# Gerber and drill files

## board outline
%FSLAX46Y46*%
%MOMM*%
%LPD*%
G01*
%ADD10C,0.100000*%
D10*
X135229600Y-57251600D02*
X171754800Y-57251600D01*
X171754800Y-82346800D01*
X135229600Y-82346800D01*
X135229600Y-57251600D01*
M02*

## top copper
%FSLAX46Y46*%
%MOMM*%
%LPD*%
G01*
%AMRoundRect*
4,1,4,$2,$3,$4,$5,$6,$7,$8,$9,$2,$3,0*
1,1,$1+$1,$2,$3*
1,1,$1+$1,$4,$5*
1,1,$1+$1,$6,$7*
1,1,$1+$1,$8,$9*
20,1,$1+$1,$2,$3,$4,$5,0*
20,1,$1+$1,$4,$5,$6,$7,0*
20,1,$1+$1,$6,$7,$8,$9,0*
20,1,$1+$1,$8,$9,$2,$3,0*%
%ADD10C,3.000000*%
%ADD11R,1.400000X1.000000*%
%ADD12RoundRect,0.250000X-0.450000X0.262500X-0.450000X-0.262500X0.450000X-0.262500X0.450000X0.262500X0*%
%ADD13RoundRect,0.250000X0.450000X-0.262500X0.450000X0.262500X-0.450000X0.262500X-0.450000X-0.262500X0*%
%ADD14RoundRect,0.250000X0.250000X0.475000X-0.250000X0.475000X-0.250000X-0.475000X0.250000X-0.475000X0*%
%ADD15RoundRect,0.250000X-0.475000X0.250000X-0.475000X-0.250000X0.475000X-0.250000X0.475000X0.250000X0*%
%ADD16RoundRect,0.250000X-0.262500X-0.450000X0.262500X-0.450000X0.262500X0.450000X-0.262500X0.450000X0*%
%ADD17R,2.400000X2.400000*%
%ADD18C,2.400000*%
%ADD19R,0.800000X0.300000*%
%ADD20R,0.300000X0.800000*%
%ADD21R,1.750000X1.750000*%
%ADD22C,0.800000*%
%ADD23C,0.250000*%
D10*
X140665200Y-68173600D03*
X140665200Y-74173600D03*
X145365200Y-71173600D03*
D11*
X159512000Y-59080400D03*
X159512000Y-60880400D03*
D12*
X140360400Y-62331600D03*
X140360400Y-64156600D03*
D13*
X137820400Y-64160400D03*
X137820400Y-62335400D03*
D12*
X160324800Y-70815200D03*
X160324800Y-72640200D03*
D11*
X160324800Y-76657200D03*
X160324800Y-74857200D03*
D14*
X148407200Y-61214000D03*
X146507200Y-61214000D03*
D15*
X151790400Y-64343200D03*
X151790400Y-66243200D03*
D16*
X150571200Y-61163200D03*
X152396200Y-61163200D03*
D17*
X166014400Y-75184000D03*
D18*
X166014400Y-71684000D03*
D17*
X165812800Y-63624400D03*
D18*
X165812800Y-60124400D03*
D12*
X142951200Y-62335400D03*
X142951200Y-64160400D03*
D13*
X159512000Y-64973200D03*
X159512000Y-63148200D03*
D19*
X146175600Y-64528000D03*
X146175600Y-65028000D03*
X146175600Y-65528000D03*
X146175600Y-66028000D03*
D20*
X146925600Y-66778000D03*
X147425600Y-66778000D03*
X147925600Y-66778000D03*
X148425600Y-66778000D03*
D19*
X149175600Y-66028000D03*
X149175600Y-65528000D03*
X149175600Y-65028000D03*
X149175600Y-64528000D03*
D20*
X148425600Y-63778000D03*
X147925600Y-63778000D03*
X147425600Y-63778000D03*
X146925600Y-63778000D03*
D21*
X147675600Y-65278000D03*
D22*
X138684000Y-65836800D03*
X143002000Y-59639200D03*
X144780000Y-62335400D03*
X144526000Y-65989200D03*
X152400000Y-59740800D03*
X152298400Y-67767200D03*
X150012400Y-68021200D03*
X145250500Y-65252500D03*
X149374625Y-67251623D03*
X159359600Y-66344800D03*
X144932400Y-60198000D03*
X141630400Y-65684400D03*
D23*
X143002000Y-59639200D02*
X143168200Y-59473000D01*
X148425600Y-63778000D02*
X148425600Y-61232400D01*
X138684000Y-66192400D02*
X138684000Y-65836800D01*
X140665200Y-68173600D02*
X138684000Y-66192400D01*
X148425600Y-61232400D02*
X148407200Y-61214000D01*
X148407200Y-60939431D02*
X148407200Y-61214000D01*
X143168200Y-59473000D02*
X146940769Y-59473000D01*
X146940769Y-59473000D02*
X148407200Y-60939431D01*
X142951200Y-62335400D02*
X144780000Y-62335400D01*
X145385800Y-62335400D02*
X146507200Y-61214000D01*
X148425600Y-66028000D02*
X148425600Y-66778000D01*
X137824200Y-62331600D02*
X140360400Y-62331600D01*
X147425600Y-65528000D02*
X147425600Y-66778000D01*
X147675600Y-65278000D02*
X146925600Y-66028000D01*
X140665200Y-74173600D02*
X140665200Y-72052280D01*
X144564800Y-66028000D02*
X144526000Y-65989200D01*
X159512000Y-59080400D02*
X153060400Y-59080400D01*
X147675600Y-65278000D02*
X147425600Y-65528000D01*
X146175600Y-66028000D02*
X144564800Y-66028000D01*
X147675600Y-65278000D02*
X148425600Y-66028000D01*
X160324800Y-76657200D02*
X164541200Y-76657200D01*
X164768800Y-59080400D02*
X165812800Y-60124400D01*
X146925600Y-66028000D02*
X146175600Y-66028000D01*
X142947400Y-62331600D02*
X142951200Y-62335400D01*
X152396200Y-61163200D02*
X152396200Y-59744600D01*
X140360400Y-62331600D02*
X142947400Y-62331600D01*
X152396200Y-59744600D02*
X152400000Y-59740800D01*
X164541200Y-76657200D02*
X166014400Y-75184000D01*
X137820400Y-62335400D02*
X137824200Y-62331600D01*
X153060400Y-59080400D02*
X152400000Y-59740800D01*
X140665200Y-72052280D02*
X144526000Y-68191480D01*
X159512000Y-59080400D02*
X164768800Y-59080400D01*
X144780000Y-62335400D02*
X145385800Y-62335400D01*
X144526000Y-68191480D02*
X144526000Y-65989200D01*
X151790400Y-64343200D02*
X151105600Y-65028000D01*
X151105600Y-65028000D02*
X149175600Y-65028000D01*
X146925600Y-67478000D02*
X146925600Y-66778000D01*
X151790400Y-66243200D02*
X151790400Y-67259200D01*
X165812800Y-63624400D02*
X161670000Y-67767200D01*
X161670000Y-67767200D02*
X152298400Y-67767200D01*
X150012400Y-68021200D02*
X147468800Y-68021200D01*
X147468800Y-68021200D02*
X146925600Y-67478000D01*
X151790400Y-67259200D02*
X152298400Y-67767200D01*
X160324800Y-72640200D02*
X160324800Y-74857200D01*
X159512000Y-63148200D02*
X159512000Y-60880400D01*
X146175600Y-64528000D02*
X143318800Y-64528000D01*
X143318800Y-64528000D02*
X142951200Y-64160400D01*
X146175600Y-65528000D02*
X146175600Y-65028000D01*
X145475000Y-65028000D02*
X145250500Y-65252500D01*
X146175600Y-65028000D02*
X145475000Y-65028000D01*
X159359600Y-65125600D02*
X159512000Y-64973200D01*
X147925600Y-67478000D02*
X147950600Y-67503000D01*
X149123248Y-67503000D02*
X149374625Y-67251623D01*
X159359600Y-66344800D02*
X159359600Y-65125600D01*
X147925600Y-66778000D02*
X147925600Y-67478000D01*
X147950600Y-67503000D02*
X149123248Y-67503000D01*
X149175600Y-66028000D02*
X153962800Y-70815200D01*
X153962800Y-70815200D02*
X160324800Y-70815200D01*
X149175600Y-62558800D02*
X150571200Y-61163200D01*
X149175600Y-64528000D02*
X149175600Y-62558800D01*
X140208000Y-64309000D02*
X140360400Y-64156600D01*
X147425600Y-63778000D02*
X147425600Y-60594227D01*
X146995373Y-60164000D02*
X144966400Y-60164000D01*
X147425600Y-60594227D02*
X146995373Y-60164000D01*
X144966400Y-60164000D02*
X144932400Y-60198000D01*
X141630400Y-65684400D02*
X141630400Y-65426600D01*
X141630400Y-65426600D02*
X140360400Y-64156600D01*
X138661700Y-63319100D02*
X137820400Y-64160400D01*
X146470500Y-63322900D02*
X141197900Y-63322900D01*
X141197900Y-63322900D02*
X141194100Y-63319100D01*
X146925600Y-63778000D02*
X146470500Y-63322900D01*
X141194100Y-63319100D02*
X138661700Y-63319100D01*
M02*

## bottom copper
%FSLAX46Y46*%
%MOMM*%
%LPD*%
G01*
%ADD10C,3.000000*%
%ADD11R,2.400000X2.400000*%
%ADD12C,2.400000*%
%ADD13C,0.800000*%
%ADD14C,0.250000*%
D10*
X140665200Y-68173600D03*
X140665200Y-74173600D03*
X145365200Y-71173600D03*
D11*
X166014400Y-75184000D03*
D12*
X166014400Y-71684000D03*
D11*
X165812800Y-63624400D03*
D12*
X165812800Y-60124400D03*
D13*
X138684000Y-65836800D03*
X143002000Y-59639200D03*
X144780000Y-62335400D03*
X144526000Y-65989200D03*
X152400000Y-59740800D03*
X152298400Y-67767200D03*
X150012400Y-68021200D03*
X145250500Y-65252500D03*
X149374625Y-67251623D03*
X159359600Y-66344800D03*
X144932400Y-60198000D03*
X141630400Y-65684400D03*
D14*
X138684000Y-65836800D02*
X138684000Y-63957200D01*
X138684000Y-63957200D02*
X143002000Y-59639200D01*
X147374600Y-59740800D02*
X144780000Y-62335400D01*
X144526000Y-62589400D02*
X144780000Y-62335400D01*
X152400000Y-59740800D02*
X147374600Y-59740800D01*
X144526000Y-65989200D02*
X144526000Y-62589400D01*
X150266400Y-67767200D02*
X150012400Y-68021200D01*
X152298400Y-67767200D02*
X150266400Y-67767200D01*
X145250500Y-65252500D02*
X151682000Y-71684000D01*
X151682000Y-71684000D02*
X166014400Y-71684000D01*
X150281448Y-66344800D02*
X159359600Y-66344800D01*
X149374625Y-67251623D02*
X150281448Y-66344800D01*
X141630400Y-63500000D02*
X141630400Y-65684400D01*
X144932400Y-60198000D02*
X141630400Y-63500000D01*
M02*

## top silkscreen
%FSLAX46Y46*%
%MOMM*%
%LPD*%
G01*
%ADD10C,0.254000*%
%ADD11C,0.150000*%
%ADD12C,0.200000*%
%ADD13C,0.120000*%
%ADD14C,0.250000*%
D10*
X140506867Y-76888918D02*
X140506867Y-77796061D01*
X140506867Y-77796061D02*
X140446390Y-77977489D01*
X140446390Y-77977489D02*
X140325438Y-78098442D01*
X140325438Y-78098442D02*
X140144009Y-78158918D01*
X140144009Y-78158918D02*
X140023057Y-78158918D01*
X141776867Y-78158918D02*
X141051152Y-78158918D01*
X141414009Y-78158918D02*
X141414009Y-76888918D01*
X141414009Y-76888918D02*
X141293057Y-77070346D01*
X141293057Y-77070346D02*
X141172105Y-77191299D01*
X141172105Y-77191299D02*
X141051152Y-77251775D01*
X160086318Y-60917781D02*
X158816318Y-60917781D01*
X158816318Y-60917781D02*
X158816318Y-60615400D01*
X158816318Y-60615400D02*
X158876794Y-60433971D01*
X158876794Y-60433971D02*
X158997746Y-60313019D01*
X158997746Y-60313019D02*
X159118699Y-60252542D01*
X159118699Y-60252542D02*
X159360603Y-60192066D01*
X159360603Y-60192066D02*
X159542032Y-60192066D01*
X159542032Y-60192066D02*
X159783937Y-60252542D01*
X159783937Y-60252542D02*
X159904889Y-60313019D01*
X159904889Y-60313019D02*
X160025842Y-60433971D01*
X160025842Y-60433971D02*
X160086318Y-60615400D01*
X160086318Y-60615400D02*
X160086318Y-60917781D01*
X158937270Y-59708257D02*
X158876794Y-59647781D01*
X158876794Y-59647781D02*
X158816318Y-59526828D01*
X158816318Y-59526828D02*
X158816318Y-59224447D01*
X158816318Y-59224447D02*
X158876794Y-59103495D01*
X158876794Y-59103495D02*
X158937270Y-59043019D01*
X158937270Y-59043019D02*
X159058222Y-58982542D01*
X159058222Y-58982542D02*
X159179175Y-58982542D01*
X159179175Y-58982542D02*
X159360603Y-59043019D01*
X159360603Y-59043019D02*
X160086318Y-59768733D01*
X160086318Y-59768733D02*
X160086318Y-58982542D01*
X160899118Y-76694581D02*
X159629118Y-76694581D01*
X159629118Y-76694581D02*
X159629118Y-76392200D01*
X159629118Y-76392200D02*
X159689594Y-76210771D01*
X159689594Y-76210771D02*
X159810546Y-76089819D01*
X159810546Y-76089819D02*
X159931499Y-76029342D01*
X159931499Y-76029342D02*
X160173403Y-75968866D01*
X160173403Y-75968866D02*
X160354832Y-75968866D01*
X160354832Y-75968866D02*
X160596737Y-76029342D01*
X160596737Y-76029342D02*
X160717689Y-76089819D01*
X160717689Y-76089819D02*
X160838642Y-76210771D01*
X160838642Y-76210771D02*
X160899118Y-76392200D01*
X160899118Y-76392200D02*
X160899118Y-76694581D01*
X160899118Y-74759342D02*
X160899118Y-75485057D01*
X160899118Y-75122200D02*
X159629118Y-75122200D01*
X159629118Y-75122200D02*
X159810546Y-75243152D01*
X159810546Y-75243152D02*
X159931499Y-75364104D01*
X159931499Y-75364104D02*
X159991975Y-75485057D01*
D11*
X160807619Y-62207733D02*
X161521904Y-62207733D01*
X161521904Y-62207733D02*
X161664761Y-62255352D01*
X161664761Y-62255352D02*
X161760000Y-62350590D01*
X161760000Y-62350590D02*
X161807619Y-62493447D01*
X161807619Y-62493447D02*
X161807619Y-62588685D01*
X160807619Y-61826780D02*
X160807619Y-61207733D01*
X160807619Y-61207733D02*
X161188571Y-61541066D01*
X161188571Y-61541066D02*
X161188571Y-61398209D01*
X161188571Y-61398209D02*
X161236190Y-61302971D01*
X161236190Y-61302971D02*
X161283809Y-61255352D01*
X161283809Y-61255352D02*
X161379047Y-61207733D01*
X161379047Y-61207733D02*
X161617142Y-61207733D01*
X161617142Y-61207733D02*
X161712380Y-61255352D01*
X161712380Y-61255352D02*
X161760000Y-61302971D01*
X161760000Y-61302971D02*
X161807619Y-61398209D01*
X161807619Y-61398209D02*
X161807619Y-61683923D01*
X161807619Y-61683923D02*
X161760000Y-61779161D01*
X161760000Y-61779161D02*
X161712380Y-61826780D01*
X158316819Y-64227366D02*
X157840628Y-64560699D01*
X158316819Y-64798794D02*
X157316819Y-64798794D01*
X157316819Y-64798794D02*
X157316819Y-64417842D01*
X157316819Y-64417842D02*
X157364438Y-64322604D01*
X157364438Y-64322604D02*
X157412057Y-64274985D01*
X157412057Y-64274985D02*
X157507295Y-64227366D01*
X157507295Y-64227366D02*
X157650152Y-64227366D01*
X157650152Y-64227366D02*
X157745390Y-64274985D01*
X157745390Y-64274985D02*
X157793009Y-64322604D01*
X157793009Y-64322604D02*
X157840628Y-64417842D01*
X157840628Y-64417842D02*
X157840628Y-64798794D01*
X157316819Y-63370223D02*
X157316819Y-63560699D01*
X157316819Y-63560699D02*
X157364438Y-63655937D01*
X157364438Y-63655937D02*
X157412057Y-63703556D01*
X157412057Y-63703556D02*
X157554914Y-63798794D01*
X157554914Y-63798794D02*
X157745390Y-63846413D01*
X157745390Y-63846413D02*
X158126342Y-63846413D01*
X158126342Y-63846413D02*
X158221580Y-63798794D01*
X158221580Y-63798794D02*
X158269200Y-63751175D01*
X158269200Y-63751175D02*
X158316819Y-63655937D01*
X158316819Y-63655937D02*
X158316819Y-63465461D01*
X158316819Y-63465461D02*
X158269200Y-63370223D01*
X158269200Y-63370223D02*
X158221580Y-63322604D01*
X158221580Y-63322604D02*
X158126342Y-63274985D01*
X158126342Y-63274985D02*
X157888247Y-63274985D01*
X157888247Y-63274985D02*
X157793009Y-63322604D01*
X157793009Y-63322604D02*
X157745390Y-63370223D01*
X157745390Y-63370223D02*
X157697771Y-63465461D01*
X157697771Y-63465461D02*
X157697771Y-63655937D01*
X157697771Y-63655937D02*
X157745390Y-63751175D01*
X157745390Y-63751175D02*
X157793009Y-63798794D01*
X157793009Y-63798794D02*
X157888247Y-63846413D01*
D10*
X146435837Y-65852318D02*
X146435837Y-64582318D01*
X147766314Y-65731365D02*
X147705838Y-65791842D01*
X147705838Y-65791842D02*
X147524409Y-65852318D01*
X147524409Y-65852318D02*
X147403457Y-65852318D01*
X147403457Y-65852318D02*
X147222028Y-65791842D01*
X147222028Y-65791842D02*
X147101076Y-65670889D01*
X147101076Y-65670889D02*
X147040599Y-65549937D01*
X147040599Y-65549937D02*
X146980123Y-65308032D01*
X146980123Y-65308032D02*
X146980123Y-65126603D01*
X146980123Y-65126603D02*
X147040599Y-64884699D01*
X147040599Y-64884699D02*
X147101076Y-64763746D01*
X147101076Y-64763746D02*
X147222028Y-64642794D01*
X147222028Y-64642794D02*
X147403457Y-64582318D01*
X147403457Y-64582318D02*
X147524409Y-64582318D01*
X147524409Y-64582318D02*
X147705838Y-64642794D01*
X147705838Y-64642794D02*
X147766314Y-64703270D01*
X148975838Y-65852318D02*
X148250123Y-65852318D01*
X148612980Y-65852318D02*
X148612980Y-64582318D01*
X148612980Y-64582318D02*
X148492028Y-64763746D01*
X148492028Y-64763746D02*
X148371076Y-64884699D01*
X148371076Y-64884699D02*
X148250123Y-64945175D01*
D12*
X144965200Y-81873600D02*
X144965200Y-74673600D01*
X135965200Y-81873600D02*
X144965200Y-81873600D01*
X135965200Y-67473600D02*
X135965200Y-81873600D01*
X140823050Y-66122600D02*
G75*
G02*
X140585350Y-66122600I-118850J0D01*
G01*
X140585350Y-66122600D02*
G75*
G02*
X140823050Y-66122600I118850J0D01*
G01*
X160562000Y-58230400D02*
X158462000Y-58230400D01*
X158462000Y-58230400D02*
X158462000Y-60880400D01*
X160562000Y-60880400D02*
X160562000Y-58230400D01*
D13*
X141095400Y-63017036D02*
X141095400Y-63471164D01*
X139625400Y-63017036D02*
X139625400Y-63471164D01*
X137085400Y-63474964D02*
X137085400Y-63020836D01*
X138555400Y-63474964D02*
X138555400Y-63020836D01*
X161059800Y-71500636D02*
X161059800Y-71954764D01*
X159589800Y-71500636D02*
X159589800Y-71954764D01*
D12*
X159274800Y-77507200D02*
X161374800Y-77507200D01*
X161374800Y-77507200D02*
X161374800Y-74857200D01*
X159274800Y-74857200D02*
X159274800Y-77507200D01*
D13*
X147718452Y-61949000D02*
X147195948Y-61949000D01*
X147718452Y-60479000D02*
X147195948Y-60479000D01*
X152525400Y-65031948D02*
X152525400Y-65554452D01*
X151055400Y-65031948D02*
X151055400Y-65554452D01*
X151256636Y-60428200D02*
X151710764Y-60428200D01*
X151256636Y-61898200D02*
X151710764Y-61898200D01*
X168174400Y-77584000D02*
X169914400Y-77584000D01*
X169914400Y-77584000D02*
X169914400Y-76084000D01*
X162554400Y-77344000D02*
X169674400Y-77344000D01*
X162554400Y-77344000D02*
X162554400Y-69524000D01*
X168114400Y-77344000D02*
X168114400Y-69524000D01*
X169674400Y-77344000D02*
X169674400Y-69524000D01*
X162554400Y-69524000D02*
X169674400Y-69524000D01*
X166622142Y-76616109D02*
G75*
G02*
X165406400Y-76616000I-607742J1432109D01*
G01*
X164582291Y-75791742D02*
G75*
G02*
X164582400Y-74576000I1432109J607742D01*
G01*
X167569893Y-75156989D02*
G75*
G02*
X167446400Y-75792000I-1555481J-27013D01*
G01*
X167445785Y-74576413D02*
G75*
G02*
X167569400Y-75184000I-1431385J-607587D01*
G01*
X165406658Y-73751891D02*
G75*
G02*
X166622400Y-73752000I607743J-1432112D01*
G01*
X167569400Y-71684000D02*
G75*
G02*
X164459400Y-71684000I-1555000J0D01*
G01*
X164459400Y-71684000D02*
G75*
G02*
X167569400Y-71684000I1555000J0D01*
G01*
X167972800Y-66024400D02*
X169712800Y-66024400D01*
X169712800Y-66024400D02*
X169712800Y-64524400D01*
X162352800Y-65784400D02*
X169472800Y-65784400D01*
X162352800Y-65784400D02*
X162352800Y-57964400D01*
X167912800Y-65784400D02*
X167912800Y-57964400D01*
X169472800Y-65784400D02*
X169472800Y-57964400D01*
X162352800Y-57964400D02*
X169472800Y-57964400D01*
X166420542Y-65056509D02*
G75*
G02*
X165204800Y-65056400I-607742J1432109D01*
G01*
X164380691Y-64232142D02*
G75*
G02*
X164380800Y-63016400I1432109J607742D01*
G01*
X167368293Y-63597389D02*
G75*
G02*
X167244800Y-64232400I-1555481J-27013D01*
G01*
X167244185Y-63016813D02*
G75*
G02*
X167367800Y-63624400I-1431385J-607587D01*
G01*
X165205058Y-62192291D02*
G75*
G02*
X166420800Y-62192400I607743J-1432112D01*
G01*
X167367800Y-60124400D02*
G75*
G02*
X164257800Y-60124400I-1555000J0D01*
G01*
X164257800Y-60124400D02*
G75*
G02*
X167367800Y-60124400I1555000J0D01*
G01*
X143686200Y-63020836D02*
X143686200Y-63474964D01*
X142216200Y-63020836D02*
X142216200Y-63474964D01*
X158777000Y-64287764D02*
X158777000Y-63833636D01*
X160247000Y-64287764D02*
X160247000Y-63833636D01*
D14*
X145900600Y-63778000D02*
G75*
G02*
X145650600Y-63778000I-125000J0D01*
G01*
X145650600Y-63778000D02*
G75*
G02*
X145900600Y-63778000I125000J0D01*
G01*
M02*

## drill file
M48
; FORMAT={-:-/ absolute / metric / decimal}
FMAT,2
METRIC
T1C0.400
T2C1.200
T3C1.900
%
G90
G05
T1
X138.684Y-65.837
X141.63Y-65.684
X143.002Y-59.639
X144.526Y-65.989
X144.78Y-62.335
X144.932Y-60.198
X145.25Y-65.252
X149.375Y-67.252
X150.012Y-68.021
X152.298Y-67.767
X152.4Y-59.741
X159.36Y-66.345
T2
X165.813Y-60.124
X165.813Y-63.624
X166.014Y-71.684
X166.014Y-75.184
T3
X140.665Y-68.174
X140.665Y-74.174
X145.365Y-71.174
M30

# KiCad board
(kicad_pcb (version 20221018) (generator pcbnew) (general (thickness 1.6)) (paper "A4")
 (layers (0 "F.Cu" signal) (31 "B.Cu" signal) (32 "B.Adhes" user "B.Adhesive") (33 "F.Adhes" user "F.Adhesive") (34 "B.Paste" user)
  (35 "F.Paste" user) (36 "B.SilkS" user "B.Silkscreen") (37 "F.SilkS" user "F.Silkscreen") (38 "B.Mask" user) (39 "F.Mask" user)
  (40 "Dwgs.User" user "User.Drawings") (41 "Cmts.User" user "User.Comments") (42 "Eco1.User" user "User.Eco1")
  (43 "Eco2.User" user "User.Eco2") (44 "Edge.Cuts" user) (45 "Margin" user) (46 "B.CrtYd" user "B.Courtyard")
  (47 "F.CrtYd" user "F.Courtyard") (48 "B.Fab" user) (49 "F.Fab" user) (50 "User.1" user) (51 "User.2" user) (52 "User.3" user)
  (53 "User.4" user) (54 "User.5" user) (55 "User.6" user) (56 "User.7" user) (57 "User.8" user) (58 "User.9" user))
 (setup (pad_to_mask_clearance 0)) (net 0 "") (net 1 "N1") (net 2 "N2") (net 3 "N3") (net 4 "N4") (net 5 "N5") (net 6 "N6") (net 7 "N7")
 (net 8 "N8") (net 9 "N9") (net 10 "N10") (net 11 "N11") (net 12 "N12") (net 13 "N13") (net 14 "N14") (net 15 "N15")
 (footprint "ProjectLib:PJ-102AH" (layer "F.Cu") (at 144.9652 71.1736 180)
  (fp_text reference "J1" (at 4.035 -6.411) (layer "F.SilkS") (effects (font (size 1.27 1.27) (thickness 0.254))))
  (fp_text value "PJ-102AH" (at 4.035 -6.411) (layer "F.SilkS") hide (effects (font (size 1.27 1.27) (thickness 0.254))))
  (fp_line (start 0 -10.7) (end 0 -3.5) (stroke (width 0.2) (type solid)) (layer "F.SilkS"))
  (fp_line (start 9 -10.7) (end 0 -10.7) (stroke (width 0.2) (type solid)) (layer "F.SilkS"))
  (fp_line (start 9 3.7) (end 9 -10.7) (stroke (width 0.2) (type solid)) (layer "F.SilkS"))
  (fp_circle (center 4.261 5.051) (end 4.261 5.16985) (stroke (width 0.2) (type solid)) (fill none) (layer "F.SilkS"))
  (pad "1" thru_hole circle (at 4.3 3 180) (size 3 3) (drill 1.9) (layers "*.Cu" "*.Mask") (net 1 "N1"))
  (pad "2" thru_hole circle (at 4.3 -3 180) (size 3 3) (drill 1.9) (layers "*.Cu" "*.Mask") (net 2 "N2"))
  (pad "3" thru_hole circle (at -0.4 0 180) (size 3 3) (drill 1.9) (layers "*.Cu" "*.Mask") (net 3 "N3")))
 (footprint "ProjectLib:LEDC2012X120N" (layer "F.Cu") (at 159.512 59.9804 -90)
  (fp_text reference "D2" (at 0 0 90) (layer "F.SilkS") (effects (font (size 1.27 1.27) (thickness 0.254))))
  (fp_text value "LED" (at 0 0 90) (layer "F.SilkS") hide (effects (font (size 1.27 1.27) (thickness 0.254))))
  (fp_line (start -1.75 -1.05) (end -1.75 1.05) (stroke (width 0.2) (type solid)) (layer "F.SilkS"))
  (fp_line (start -1.75 1.05) (end 0.9 1.05) (stroke (width 0.2) (type solid)) (layer "F.SilkS"))
  (fp_line (start 0.9 -1.05) (end -1.75 -1.05) (stroke (width 0.2) (type solid)) (layer "F.SilkS"))
  (pad "1" smd rect (at -0.9 0 270) (size 1 1.4) (layers "F.Cu" "F.Paste" "F.Mask") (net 2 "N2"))
  (pad "2" smd rect (at 0.9 0 270) (size 1 1.4) (layers "F.Cu" "F.Paste" "F.Mask") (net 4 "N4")))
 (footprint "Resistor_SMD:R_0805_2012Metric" (layer "F.Cu") (at 140.3604 63.2441 -90)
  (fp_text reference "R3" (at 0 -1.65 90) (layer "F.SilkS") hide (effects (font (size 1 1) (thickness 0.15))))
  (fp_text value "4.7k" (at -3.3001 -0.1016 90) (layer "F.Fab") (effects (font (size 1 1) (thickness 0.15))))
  (fp_line (start -0.227064 -0.735) (end 0.227064 -0.735) (stroke (width 0.12) (type solid)) (layer "F.SilkS"))
  (fp_line (start -0.227064 0.735) (end 0.227064 0.735) (stroke (width 0.12) (type solid)) (layer "F.SilkS"))
  (pad "1" smd roundrect (at -0.9125 0 270) (size 1.025 1.4) (layers "F.Cu" "F.Paste" "F.Mask") (roundrect_rratio 0.243902) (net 2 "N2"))
  (pad "2" smd roundrect (at 0.9125 0 270) (size 1.025 1.4) (layers "F.Cu" "F.Paste" "F.Mask") (roundrect_rratio 0.243902) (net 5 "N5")))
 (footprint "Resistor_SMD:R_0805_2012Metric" (layer "F.Cu") (at 137.8204 63.2479 90)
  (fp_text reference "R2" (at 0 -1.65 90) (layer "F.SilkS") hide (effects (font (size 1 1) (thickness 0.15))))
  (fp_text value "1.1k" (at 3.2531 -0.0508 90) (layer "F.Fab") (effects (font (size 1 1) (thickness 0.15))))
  (fp_line (start -0.227064 -0.735) (end 0.227064 -0.735) (stroke (width 0.12) (type solid)) (layer "F.SilkS"))
  (fp_line (start -0.227064 0.735) (end 0.227064 0.735) (stroke (width 0.12) (type solid)) (layer "F.SilkS"))
  (pad "1" smd roundrect (at -0.9125 0 90) (size 1.025 1.4) (layers "F.Cu" "F.Paste" "F.Mask") (roundrect_rratio 0.243902) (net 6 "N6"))
  (pad "2" smd roundrect (at 0.9125 0 90) (size 1.025 1.4) (layers "F.Cu" "F.Paste" "F.Mask") (roundrect_rratio 0.243902) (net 2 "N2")))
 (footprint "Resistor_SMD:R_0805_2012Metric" (layer "F.Cu") (at 160.3248 71.7277 -90)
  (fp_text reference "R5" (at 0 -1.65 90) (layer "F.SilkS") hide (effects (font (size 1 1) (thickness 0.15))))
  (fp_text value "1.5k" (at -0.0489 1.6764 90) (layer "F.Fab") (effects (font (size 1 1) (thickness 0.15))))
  (fp_line (start -0.227064 -0.735) (end 0.227064 -0.735) (stroke (width 0.12) (type solid)) (layer "F.SilkS"))
  (fp_line (start -0.227064 0.735) (end 0.227064 0.735) (stroke (width 0.12) (type solid)) (layer "F.SilkS"))
  (pad "1" smd roundrect (at -0.9125 0 270) (size 1.025 1.4) (layers "F.Cu" "F.Paste" "F.Mask") (roundrect_rratio 0.243902) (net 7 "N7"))
  (pad "2" smd roundrect (at 0.9125 0 270) (size 1.025 1.4) (layers "F.Cu" "F.Paste" "F.Mask") (roundrect_rratio 0.243902) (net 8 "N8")))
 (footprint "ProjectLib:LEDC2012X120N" (layer "F.Cu") (at 160.3248 75.7572 90)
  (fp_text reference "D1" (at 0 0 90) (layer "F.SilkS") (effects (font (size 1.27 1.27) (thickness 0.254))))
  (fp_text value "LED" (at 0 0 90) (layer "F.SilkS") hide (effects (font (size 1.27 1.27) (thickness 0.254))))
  (fp_line (start -1.75 -1.05) (end -1.75 1.05) (stroke (width 0.2) (type solid)) (layer "F.SilkS"))
  (fp_line (start -1.75 1.05) (end 0.9 1.05) (stroke (width 0.2) (type solid)) (layer "F.SilkS"))
  (fp_line (start 0.9 -1.05) (end -1.75 -1.05) (stroke (width 0.2) (type solid)) (layer "F.SilkS"))
  (pad "1" smd rect (at -0.9 0 90) (size 1 1.4) (layers "F.Cu" "F.Paste" "F.Mask") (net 2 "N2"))
  (pad "2" smd rect (at 0.9 0 90) (size 1 1.4) (layers "F.Cu" "F.Paste" "F.Mask") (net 8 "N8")))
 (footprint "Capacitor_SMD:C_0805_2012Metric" (layer "F.Cu") (at 147.4572 61.214 180)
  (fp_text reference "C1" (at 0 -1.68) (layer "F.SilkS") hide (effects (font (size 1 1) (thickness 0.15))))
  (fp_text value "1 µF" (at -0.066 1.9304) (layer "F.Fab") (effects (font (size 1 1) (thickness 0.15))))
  (fp_line (start -0.261252 -0.735) (end 0.261252 -0.735) (stroke (width 0.12) (type solid)) (layer "F.SilkS"))
  (fp_line (start -0.261252 0.735) (end 0.261252 0.735) (stroke (width 0.12) (type solid)) (layer "F.SilkS"))
  (pad "1" smd roundrect (at -0.95 0 180) (size 1 1.45) (layers "F.Cu" "F.Paste" "F.Mask") (roundrect_rratio 0.25) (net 1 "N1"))
  (pad "2" smd roundrect (at 0.95 0 180) (size 1 1.45) (layers "F.Cu" "F.Paste" "F.Mask") (roundrect_rratio 0.25) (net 2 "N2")))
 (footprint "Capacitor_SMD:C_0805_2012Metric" (layer "F.Cu") (at 151.7904 65.2932 -90)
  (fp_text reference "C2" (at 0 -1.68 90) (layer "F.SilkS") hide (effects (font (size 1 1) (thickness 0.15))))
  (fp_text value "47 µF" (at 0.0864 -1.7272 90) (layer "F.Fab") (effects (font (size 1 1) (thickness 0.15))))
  (fp_line (start -0.261252 -0.735) (end 0.261252 -0.735) (stroke (width 0.12) (type solid)) (layer "F.SilkS"))
  (fp_line (start -0.261252 0.735) (end 0.261252 0.735) (stroke (width 0.12) (type solid)) (layer "F.SilkS"))
  (pad "1" smd roundrect (at -0.95 0 270) (size 1 1.45) (layers "F.Cu" "F.Paste" "F.Mask") (roundrect_rratio 0.25) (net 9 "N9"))
  (pad "2" smd roundrect (at 0.95 0 270) (size 1 1.45) (layers "F.Cu" "F.Paste" "F.Mask") (roundrect_rratio 0.25) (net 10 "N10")))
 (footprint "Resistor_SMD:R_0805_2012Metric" (layer "F.Cu") (at 151.4837 61.1632)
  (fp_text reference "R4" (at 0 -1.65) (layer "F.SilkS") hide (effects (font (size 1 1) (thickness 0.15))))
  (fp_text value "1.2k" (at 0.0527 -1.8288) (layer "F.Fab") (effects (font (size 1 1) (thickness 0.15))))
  (fp_line (start -0.227064 -0.735) (end 0.227064 -0.735) (stroke (width 0.12) (type solid)) (layer "F.SilkS"))
  (fp_line (start -0.227064 0.735) (end 0.227064 0.735) (stroke (width 0.12) (type solid)) (layer "F.SilkS"))
  (pad "1" smd roundrect (at -0.9125 0) (size 1.025 1.4) (layers "F.Cu" "F.Paste" "F.Mask") (roundrect_rratio 0.243902) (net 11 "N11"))
  (pad "2" smd roundrect (at 0.9125 0) (size 1.025 1.4) (layers "F.Cu" "F.Paste" "F.Mask") (roundrect_rratio 0.243902) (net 2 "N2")))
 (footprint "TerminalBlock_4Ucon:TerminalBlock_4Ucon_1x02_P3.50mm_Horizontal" (layer "F.Cu") (at 166.0144 75.184 90)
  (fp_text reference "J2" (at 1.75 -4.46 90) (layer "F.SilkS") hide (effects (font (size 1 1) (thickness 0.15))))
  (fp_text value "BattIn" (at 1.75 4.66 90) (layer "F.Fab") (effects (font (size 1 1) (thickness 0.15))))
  (fp_line (start -2.4 2.16) (end -2.4 3.9) (stroke (width 0.12) (type solid)) (layer "F.SilkS"))
  (fp_line (start -2.4 3.9) (end -0.9 3.9) (stroke (width 0.12) (type solid)) (layer "F.SilkS"))
  (fp_line (start -2.16 -3.46) (end -2.16 3.66) (stroke (width 0.12) (type solid)) (layer "F.SilkS"))
  (fp_line (start -2.16 -3.46) (end 5.66 -3.46) (stroke (width 0.12) (type solid)) (layer "F.SilkS"))
  (fp_line (start -2.16 2.1) (end 5.66 2.1) (stroke (width 0.12) (type solid)) (layer "F.SilkS"))
  (fp_line (start -2.16 3.66) (end 5.66 3.66) (stroke (width 0.12) (type solid)) (layer "F.SilkS"))
  (fp_line (start 5.66 -3.46) (end 5.66 3.66) (stroke (width 0.12) (type solid)) (layer "F.SilkS"))
  (fp_arc (start -1.432109 0.607742) (mid -1.555727 -0.00014) (end -1.432 -0.608) (stroke (width 0.12) (type solid)) (layer "F.SilkS"))
  (fp_arc (start -0.607742 -1.432109) (mid 0.00014 -1.555727) (end 0.608 -1.432) (stroke (width 0.12) (type solid)) (layer "F.SilkS"))
  (fp_arc (start 0.027011 1.555493) (mid -0.296984 1.527118) (end -0.608 1.432) (stroke (width 0.12) (type solid)) (layer "F.SilkS"))
  (fp_arc (start 0.607587 1.431385) (mid 0.310017 1.523783) (end 0 1.555) (stroke (width 0.12) (type solid)) (layer "F.SilkS"))
  (fp_arc (start 1.432109 -0.607742) (mid 1.555727 0.00014) (end 1.432 0.608) (stroke (width 0.12) (type solid)) (layer "F.SilkS"))
  (fp_circle (center 3.5 0) (end 5.055 0) (stroke (width 0.12) (type solid)) (fill none) (layer "F.SilkS"))
  (pad "1" thru_hole rect (at 0 0 90) (size 2.4 2.4) (drill 1.2) (layers "*.Cu" "*.Mask") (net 2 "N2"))
  (pad "2" thru_hole circle (at 3.5 0 90) (size 2.4 2.4) (drill 1.2) (layers "*.Cu" "*.Mask") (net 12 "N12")))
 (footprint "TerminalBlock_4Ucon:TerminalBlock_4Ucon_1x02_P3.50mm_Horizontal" (layer "F.Cu") (at 165.8128 63.6244 90)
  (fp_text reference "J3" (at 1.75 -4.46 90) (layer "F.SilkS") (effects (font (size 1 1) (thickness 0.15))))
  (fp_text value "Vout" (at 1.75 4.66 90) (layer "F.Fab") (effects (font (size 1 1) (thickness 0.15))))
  (fp_line (start -2.4 2.16) (end -2.4 3.9) (stroke (width 0.12) (type solid)) (layer "F.SilkS"))
  (fp_line (start -2.4 3.9) (end -0.9 3.9) (stroke (width 0.12) (type solid)) (layer "F.SilkS"))
  (fp_line (start -2.16 -3.46) (end -2.16 3.66) (stroke (width 0.12) (type solid)) (layer "F.SilkS"))
  (fp_line (start -2.16 -3.46) (end 5.66 -3.46) (stroke (width 0.12) (type solid)) (layer "F.SilkS"))
  (fp_line (start -2.16 2.1) (end 5.66 2.1) (stroke (width 0.12) (type solid)) (layer "F.SilkS"))
  (fp_line (start -2.16 3.66) (end 5.66 3.66) (stroke (width 0.12) (type solid)) (layer "F.SilkS"))
  (fp_line (start 5.66 -3.46) (end 5.66 3.66) (stroke (width 0.12) (type solid)) (layer "F.SilkS"))
  (fp_arc (start -1.432109 0.607742) (mid -1.555727 -0.00014) (end -1.432 -0.608) (stroke (width 0.12) (type solid)) (layer "F.SilkS"))
  (fp_arc (start -0.607742 -1.432109) (mid 0.00014 -1.555727) (end 0.608 -1.432) (stroke (width 0.12) (type solid)) (layer "F.SilkS"))
  (fp_arc (start 0.027011 1.555493) (mid -0.296984 1.527118) (end -0.608 1.432) (stroke (width 0.12) (type solid)) (layer "F.SilkS"))
  (fp_arc (start 0.607587 1.431385) (mid 0.310017 1.523783) (end 0 1.555) (stroke (width 0.12) (type solid)) (layer "F.SilkS"))
  (fp_arc (start 1.432109 -0.607742) (mid 1.555727 0.00014) (end 1.432 0.608) (stroke (width 0.12) (type solid)) (layer "F.SilkS"))
  (fp_circle (center 3.5 0) (end 5.055 0) (stroke (width 0.12) (type solid)) (fill none) (layer "F.SilkS"))
  (pad "1" thru_hole rect (at 0 0 90) (size 2.4 2.4) (drill 1.2) (layers "*.Cu" "*.Mask") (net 10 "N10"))
  (pad "2" thru_hole circle (at 3.5 0 90) (size 2.4 2.4) (drill 1.2) (layers "*.Cu" "*.Mask") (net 2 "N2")))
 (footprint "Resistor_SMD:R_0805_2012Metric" (layer "F.Cu") (at 142.9512 63.2479 -90)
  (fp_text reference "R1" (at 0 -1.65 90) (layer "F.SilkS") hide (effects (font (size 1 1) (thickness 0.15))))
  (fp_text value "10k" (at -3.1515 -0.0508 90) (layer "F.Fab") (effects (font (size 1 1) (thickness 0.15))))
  (fp_line (start -0.227064 -0.735) (end 0.227064 -0.735) (stroke (width 0.12) (type solid)) (layer "F.SilkS"))
  (fp_line (start -0.227064 0.735) (end 0.227064 0.735) (stroke (width 0.12) (type solid)) (layer "F.SilkS"))
  (pad "1" smd roundrect (at -0.9125 0 270) (size 1.025 1.4) (layers "F.Cu" "F.Paste" "F.Mask") (roundrect_rratio 0.243902) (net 2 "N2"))
  (pad "2" smd roundrect (at 0.9125 0 270) (size 1.025 1.4) (layers "F.Cu" "F.Paste" "F.Mask") (roundrect_rratio 0.243902) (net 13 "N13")))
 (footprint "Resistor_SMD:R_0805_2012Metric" (layer "F.Cu") (at 159.512 64.0607 90)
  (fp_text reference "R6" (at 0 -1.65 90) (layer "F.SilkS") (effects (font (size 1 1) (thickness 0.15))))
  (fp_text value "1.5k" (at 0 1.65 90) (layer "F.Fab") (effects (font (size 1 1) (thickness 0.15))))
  (fp_line (start -0.227064 -0.735) (end 0.227064 -0.735) (stroke (width 0.12) (type solid)) (layer "F.SilkS"))
  (fp_line (start -0.227064 0.735) (end 0.227064 0.735) (stroke (width 0.12) (type solid)) (layer "F.SilkS"))
  (pad "1" smd roundrect (at -0.9125 0 90) (size 1.025 1.4) (layers "F.Cu" "F.Paste" "F.Mask") (roundrect_rratio 0.243902) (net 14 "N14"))
  (pad "2" smd roundrect (at 0.9125 0 90) (size 1.025 1.4) (layers "F.Cu" "F.Paste" "F.Mask") (roundrect_rratio 0.243902) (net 4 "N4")))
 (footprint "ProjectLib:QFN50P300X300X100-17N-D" (layer "F.Cu") (at 147.6756 65.278)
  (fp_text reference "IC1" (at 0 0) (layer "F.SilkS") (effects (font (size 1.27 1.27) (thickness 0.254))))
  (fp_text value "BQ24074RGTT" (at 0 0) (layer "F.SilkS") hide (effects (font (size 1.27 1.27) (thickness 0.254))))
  (fp_circle (center -1.9 -1.5) (end -1.9 -1.375) (stroke (width 0.25) (type solid)) (fill none) (layer "F.SilkS"))
  (pad "1" smd rect (at -1.5 -0.75 90) (size 0.3 0.8) (layers "F.Cu" "F.Paste" "F.Mask") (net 13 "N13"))
  (pad "2" smd rect (at -1.5 -0.25 90) (size 0.3 0.8) (layers "F.Cu" "F.Paste" "F.Mask") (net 12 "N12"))
  (pad "3" smd rect (at -1.5 0.25 90) (size 0.3 0.8) (layers "F.Cu" "F.Paste" "F.Mask") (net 12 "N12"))
  (pad "4" smd rect (at -1.5 0.75 90) (size 0.3 0.8) (layers "F.Cu" "F.Paste" "F.Mask") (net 2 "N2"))
  (pad "5" smd rect (at -0.75 1.5) (size 0.3 0.8) (layers "F.Cu" "F.Paste" "F.Mask") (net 10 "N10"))
  (pad "6" smd rect (at -0.25 1.5) (size 0.3 0.8) (layers "F.Cu" "F.Paste" "F.Mask") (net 2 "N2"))
  (pad "7" smd rect (at 0.25 1.5) (size 0.3 0.8) (layers "F.Cu" "F.Paste" "F.Mask") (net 14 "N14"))
  (pad "8" smd rect (at 0.75 1.5) (size 0.3 0.8) (layers "F.Cu" "F.Paste" "F.Mask") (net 2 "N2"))
  (pad "9" smd rect (at 1.5 0.75 90) (size 0.3 0.8) (layers "F.Cu" "F.Paste" "F.Mask") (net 7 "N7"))
  (pad "10" smd rect (at 1.5 0.25 90) (size 0.3 0.8) (layers "F.Cu" "F.Paste" "F.Mask") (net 9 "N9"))
  (pad "11" smd rect (at 1.5 -0.25 90) (size 0.3 0.8) (layers "F.Cu" "F.Paste" "F.Mask") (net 9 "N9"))
  (pad "12" smd rect (at 1.5 -0.75 90) (size 0.3 0.8) (layers "F.Cu" "F.Paste" "F.Mask") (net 11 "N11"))
  (pad "13" smd rect (at 0.75 -1.5) (size 0.3 0.8) (layers "F.Cu" "F.Paste" "F.Mask") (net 1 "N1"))
  (pad "14" smd rect (at 0.25 -1.5) (size 0.3 0.8) (layers "F.Cu" "F.Paste" "F.Mask") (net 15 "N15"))
  (pad "15" smd rect (at -0.25 -1.5) (size 0.3 0.8) (layers "F.Cu" "F.Paste" "F.Mask") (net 5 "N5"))
  (pad "16" smd rect (at -0.75 -1.5) (size 0.3 0.8) (layers "F.Cu" "F.Paste" "F.Mask") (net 6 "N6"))
  (pad "17" smd rect (at 0 0) (size 1.75 1.75) (layers "F.Cu" "F.Paste" "F.Mask") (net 2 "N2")))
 (gr_rect (start 135.2296 57.2516) (end 171.7548 82.3468) (stroke (width 0.1) (type default)) (fill none) (layer "Edge.Cuts"))
 (segment (start 143.002 59.6392) (end 143.1682 59.473) (width 0.25) (layer "F.Cu") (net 1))
 (segment (start 148.4256 63.778) (end 148.4256 61.2324) (width 0.25) (layer "F.Cu") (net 1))
 (segment (start 138.684 66.1924) (end 138.684 65.8368) (width 0.25) (layer "F.Cu") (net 1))
 (segment (start 140.6652 68.1736) (end 138.684 66.1924) (width 0.25) (layer "F.Cu") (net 1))
 (segment (start 148.4256 61.2324) (end 148.4072 61.214) (width 0.25) (layer "F.Cu") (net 1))
 (segment (start 148.4072 60.939431) (end 148.4072 61.214) (width 0.25) (layer "F.Cu") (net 1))
 (segment (start 143.1682 59.473) (end 146.940769 59.473) (width 0.25) (layer "F.Cu") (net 1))
 (segment (start 146.940769 59.473) (end 148.4072 60.939431) (width 0.25) (layer "F.Cu") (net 1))
 (via (at 138.684 65.8368) (size 0.8) (drill 0.4) (layers "F.Cu" "B.Cu") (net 1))
 (via (at 143.002 59.6392) (size 0.8) (drill 0.4) (layers "F.Cu" "B.Cu") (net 1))
 (segment (start 138.684 65.8368) (end 138.684 63.9572) (width 0.25) (layer "B.Cu") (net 1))
 (segment (start 138.684 63.9572) (end 143.002 59.6392) (width 0.25) (layer "B.Cu") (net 1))
 (segment (start 142.9512 62.3354) (end 144.78 62.3354) (width 0.25) (layer "F.Cu") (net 2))
 (segment (start 145.3858 62.3354) (end 146.5072 61.214) (width 0.25) (layer "F.Cu") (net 2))
 (segment (start 148.4256 66.028) (end 148.4256 66.778) (width 0.25) (layer "F.Cu") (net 2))
 (segment (start 137.8242 62.3316) (end 140.3604 62.3316) (width 0.25) (layer "F.Cu") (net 2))
 (segment (start 147.4256 65.528) (end 147.4256 66.778) (width 0.25) (layer "F.Cu") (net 2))
 (segment (start 147.6756 65.278) (end 146.9256 66.028) (width 0.25) (layer "F.Cu") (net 2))
 (segment (start 140.6652 74.1736) (end 140.6652 72.05228) (width 0.25) (layer "F.Cu") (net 2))
 (segment (start 144.5648 66.028) (end 144.526 65.9892) (width 0.25) (layer "F.Cu") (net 2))
 (segment (start 159.512 59.0804) (end 153.0604 59.0804) (width 0.25) (layer "F.Cu") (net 2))
 (segment (start 147.6756 65.278) (end 147.4256 65.528) (width 0.25) (layer "F.Cu") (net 2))
 (segment (start 146.1756 66.028) (end 144.5648 66.028) (width 0.25) (layer "F.Cu") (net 2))
 (segment (start 147.6756 65.278) (end 148.4256 66.028) (width 0.25) (layer "F.Cu") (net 2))
 (segment (start 160.3248 76.6572) (end 164.5412 76.6572) (width 0.25) (layer "F.Cu") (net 2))
 (segment (start 164.7688 59.0804) (end 165.8128 60.1244) (width 0.25) (layer "F.Cu") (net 2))
 (segment (start 146.9256 66.028) (end 146.1756 66.028) (width 0.25) (layer "F.Cu") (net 2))
 (segment (start 142.9474 62.3316) (end 142.9512 62.3354) (width 0.25) (layer "F.Cu") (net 2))
 (segment (start 152.3962 61.1632) (end 152.3962 59.7446) (width 0.25) (layer "F.Cu") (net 2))
 (segment (start 140.3604 62.3316) (end 142.9474 62.3316) (width 0.25) (layer "F.Cu") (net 2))
 (segment (start 152.3962 59.7446) (end 152.4 59.7408) (width 0.25) (layer "F.Cu") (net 2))
 (segment (start 164.5412 76.6572) (end 166.0144 75.184) (width 0.25) (layer "F.Cu") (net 2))
 (segment (start 137.8204 62.3354) (end 137.8242 62.3316) (width 0.25) (layer "F.Cu") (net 2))
 (segment (start 153.0604 59.0804) (end 152.4 59.7408) (width 0.25) (layer "F.Cu") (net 2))
 (segment (start 140.6652 72.05228) (end 144.526 68.19148) (width 0.25) (layer "F.Cu") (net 2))
 (segment (start 159.512 59.0804) (end 164.7688 59.0804) (width 0.25) (layer "F.Cu") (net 2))
 (segment (start 144.78 62.3354) (end 145.3858 62.3354) (width 0.25) (layer "F.Cu") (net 2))
 (segment (start 144.526 68.19148) (end 144.526 65.9892) (width 0.25) (layer "F.Cu") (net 2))
 (via (at 144.78 62.3354) (size 0.8) (drill 0.4) (layers "F.Cu" "B.Cu") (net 2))
 (via (at 144.526 65.9892) (size 0.8) (drill 0.4) (layers "F.Cu" "B.Cu") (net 2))
 (via (at 152.4 59.7408) (size 0.8) (drill 0.4) (layers "F.Cu" "B.Cu") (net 2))
 (segment (start 147.3746 59.7408) (end 144.78 62.3354) (width 0.25) (layer "B.Cu") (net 2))
 (segment (start 144.526 62.5894) (end 144.78 62.3354) (width 0.25) (layer "B.Cu") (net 2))
 (segment (start 152.4 59.7408) (end 147.3746 59.7408) (width 0.25) (layer "B.Cu") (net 2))
 (segment (start 144.526 65.9892) (end 144.526 62.5894) (width 0.25) (layer "B.Cu") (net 2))
 (segment (start 151.7904 64.3432) (end 151.1056 65.028) (width 0.25) (layer "F.Cu") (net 9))
 (segment (start 151.1056 65.028) (end 149.1756 65.028) (width 0.25) (layer "F.Cu") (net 9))
 (segment (start 146.9256 67.478) (end 146.9256 66.778) (width 0.25) (layer "F.Cu") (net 10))
 (segment (start 151.7904 66.2432) (end 151.7904 67.2592) (width 0.25) (layer "F.Cu") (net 10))
 (segment (start 165.8128 63.6244) (end 161.67 67.7672) (width 0.25) (layer "F.Cu") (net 10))
 (segment (start 161.67 67.7672) (end 152.2984 67.7672) (width 0.25) (layer "F.Cu") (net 10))
 (segment (start 150.0124 68.0212) (end 147.4688 68.0212) (width 0.25) (layer "F.Cu") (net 10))
 (segment (start 147.4688 68.0212) (end 146.9256 67.478) (width 0.25) (layer "F.Cu") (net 10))
 (segment (start 151.7904 67.2592) (end 152.2984 67.7672) (width 0.25) (layer "F.Cu") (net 10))
 (via (at 152.2984 67.7672) (size 0.8) (drill 0.4) (layers "F.Cu" "B.Cu") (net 10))
 (via (at 150.0124 68.0212) (size 0.8) (drill 0.4) (layers "F.Cu" "B.Cu") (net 10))
 (segment (start 150.2664 67.7672) (end 150.0124 68.0212) (width 0.25) (layer "B.Cu") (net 10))
 (segment (start 152.2984 67.7672) (end 150.2664 67.7672) (width 0.25) (layer "B.Cu") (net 10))
 (segment (start 160.3248 72.6402) (end 160.3248 74.8572) (width 0.25) (layer "F.Cu") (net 8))
 (segment (start 159.512 63.1482) (end 159.512 60.8804) (width 0.25) (layer "F.Cu") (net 4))
 (segment (start 146.1756 64.528) (end 143.3188 64.528) (width 0.25) (layer "F.Cu") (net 13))
 (segment (start 143.3188 64.528) (end 142.9512 64.1604) (width 0.25) (layer "F.Cu") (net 13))
 (segment (start 146.1756 65.528) (end 146.1756 65.028) (width 0.25) (layer "F.Cu") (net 12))
 (segment (start 145.475 65.028) (end 145.2505 65.2525) (width 0.25) (layer "F.Cu") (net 12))
 (segment (start 146.1756 65.028) (end 145.475 65.028) (width 0.25) (layer "F.Cu") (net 12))
 (via (at 145.2505 65.2525) (size 0.8) (drill 0.4) (layers "F.Cu" "B.Cu") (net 12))
 (segment (start 145.2505 65.2525) (end 151.682 71.684) (width 0.25) (layer "B.Cu") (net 12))
 (segment (start 151.682 71.684) (end 166.0144 71.684) (width 0.25) (layer "B.Cu") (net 12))
 (segment (start 159.3596 65.1256) (end 159.512 64.9732) (width 0.25) (layer "F.Cu") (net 14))
 (segment (start 147.9256 67.478) (end 147.9506 67.503) (width 0.25) (layer "F.Cu") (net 14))
 (segment (start 149.123248 67.503) (end 149.374625 67.251623) (width 0.25) (layer "F.Cu") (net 14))
 (segment (start 159.3596 66.3448) (end 159.3596 65.1256) (width 0.25) (layer "F.Cu") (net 14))
 (segment (start 147.9256 66.778) (end 147.9256 67.478) (width 0.25) (layer "F.Cu") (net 14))
 (segment (start 147.9506 67.503) (end 149.123248 67.503) (width 0.25) (layer "F.Cu") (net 14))
 (via (at 149.374625 67.251623) (size 0.8) (drill 0.4) (layers "F.Cu" "B.Cu") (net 14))
 (via (at 159.3596 66.3448) (size 0.8) (drill 0.4) (layers "F.Cu" "B.Cu") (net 14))
 (segment (start 150.281448 66.3448) (end 159.3596 66.3448) (width 0.25) (layer "B.Cu") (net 14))
 (segment (start 149.374625 67.251623) (end 150.281448 66.3448) (width 0.25) (layer "B.Cu") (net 14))
 (segment (start 149.1756 66.028) (end 153.9628 70.8152) (width 0.25) (layer "F.Cu") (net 7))
 (segment (start 153.9628 70.8152) (end 160.3248 70.8152) (width 0.25) (layer "F.Cu") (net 7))
 (segment (start 149.1756 62.5588) (end 150.5712 61.1632) (width 0.25) (layer "F.Cu") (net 11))
 (segment (start 149.1756 64.528) (end 149.1756 62.5588) (width 0.25) (layer "F.Cu") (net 11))
 (segment (start 140.208 64.309) (end 140.3604 64.1566) (width 0.25) (layer "F.Cu") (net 5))
 (segment (start 147.4256 63.778) (end 147.4256 60.594227) (width 0.25) (layer "F.Cu") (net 5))
 (segment (start 146.995373 60.164) (end 144.9664 60.164) (width 0.25) (layer "F.Cu") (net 5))
 (segment (start 147.4256 60.594227) (end 146.995373 60.164) (width 0.25) (layer "F.Cu") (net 5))
 (segment (start 144.9664 60.164) (end 144.9324 60.198) (width 0.25) (layer "F.Cu") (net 5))
 (segment (start 141.6304 65.6844) (end 141.6304 65.4266) (width 0.25) (layer "F.Cu") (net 5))
 (segment (start 141.6304 65.4266) (end 140.3604 64.1566) (width 0.25) (layer "F.Cu") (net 5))
 (via (at 144.9324 60.198) (size 0.8) (drill 0.4) (layers "F.Cu" "B.Cu") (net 5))
 (via (at 141.6304 65.6844) (size 0.8) (drill 0.4) (layers "F.Cu" "B.Cu") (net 5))
 (segment (start 141.6304 63.5) (end 141.6304 65.6844) (width 0.25) (layer "B.Cu") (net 5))
 (segment (start 144.9324 60.198) (end 141.6304 63.5) (width 0.25) (layer "B.Cu") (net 5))
 (segment (start 138.6617 63.3191) (end 137.8204 64.1604) (width 0.25) (layer "F.Cu") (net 6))
 (segment (start 146.4705 63.3229) (end 141.1979 63.3229) (width 0.25) (layer "F.Cu") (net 6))
 (segment (start 141.1979 63.3229) (end 141.1941 63.3191) (width 0.25) (layer "F.Cu") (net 6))
 (segment (start 146.9256 63.778) (end 146.4705 63.3229) (width 0.25) (layer "F.Cu") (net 6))
 (segment (start 141.1941 63.3191) (end 138.6617 63.3191) (width 0.25) (layer "F.Cu") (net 6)))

